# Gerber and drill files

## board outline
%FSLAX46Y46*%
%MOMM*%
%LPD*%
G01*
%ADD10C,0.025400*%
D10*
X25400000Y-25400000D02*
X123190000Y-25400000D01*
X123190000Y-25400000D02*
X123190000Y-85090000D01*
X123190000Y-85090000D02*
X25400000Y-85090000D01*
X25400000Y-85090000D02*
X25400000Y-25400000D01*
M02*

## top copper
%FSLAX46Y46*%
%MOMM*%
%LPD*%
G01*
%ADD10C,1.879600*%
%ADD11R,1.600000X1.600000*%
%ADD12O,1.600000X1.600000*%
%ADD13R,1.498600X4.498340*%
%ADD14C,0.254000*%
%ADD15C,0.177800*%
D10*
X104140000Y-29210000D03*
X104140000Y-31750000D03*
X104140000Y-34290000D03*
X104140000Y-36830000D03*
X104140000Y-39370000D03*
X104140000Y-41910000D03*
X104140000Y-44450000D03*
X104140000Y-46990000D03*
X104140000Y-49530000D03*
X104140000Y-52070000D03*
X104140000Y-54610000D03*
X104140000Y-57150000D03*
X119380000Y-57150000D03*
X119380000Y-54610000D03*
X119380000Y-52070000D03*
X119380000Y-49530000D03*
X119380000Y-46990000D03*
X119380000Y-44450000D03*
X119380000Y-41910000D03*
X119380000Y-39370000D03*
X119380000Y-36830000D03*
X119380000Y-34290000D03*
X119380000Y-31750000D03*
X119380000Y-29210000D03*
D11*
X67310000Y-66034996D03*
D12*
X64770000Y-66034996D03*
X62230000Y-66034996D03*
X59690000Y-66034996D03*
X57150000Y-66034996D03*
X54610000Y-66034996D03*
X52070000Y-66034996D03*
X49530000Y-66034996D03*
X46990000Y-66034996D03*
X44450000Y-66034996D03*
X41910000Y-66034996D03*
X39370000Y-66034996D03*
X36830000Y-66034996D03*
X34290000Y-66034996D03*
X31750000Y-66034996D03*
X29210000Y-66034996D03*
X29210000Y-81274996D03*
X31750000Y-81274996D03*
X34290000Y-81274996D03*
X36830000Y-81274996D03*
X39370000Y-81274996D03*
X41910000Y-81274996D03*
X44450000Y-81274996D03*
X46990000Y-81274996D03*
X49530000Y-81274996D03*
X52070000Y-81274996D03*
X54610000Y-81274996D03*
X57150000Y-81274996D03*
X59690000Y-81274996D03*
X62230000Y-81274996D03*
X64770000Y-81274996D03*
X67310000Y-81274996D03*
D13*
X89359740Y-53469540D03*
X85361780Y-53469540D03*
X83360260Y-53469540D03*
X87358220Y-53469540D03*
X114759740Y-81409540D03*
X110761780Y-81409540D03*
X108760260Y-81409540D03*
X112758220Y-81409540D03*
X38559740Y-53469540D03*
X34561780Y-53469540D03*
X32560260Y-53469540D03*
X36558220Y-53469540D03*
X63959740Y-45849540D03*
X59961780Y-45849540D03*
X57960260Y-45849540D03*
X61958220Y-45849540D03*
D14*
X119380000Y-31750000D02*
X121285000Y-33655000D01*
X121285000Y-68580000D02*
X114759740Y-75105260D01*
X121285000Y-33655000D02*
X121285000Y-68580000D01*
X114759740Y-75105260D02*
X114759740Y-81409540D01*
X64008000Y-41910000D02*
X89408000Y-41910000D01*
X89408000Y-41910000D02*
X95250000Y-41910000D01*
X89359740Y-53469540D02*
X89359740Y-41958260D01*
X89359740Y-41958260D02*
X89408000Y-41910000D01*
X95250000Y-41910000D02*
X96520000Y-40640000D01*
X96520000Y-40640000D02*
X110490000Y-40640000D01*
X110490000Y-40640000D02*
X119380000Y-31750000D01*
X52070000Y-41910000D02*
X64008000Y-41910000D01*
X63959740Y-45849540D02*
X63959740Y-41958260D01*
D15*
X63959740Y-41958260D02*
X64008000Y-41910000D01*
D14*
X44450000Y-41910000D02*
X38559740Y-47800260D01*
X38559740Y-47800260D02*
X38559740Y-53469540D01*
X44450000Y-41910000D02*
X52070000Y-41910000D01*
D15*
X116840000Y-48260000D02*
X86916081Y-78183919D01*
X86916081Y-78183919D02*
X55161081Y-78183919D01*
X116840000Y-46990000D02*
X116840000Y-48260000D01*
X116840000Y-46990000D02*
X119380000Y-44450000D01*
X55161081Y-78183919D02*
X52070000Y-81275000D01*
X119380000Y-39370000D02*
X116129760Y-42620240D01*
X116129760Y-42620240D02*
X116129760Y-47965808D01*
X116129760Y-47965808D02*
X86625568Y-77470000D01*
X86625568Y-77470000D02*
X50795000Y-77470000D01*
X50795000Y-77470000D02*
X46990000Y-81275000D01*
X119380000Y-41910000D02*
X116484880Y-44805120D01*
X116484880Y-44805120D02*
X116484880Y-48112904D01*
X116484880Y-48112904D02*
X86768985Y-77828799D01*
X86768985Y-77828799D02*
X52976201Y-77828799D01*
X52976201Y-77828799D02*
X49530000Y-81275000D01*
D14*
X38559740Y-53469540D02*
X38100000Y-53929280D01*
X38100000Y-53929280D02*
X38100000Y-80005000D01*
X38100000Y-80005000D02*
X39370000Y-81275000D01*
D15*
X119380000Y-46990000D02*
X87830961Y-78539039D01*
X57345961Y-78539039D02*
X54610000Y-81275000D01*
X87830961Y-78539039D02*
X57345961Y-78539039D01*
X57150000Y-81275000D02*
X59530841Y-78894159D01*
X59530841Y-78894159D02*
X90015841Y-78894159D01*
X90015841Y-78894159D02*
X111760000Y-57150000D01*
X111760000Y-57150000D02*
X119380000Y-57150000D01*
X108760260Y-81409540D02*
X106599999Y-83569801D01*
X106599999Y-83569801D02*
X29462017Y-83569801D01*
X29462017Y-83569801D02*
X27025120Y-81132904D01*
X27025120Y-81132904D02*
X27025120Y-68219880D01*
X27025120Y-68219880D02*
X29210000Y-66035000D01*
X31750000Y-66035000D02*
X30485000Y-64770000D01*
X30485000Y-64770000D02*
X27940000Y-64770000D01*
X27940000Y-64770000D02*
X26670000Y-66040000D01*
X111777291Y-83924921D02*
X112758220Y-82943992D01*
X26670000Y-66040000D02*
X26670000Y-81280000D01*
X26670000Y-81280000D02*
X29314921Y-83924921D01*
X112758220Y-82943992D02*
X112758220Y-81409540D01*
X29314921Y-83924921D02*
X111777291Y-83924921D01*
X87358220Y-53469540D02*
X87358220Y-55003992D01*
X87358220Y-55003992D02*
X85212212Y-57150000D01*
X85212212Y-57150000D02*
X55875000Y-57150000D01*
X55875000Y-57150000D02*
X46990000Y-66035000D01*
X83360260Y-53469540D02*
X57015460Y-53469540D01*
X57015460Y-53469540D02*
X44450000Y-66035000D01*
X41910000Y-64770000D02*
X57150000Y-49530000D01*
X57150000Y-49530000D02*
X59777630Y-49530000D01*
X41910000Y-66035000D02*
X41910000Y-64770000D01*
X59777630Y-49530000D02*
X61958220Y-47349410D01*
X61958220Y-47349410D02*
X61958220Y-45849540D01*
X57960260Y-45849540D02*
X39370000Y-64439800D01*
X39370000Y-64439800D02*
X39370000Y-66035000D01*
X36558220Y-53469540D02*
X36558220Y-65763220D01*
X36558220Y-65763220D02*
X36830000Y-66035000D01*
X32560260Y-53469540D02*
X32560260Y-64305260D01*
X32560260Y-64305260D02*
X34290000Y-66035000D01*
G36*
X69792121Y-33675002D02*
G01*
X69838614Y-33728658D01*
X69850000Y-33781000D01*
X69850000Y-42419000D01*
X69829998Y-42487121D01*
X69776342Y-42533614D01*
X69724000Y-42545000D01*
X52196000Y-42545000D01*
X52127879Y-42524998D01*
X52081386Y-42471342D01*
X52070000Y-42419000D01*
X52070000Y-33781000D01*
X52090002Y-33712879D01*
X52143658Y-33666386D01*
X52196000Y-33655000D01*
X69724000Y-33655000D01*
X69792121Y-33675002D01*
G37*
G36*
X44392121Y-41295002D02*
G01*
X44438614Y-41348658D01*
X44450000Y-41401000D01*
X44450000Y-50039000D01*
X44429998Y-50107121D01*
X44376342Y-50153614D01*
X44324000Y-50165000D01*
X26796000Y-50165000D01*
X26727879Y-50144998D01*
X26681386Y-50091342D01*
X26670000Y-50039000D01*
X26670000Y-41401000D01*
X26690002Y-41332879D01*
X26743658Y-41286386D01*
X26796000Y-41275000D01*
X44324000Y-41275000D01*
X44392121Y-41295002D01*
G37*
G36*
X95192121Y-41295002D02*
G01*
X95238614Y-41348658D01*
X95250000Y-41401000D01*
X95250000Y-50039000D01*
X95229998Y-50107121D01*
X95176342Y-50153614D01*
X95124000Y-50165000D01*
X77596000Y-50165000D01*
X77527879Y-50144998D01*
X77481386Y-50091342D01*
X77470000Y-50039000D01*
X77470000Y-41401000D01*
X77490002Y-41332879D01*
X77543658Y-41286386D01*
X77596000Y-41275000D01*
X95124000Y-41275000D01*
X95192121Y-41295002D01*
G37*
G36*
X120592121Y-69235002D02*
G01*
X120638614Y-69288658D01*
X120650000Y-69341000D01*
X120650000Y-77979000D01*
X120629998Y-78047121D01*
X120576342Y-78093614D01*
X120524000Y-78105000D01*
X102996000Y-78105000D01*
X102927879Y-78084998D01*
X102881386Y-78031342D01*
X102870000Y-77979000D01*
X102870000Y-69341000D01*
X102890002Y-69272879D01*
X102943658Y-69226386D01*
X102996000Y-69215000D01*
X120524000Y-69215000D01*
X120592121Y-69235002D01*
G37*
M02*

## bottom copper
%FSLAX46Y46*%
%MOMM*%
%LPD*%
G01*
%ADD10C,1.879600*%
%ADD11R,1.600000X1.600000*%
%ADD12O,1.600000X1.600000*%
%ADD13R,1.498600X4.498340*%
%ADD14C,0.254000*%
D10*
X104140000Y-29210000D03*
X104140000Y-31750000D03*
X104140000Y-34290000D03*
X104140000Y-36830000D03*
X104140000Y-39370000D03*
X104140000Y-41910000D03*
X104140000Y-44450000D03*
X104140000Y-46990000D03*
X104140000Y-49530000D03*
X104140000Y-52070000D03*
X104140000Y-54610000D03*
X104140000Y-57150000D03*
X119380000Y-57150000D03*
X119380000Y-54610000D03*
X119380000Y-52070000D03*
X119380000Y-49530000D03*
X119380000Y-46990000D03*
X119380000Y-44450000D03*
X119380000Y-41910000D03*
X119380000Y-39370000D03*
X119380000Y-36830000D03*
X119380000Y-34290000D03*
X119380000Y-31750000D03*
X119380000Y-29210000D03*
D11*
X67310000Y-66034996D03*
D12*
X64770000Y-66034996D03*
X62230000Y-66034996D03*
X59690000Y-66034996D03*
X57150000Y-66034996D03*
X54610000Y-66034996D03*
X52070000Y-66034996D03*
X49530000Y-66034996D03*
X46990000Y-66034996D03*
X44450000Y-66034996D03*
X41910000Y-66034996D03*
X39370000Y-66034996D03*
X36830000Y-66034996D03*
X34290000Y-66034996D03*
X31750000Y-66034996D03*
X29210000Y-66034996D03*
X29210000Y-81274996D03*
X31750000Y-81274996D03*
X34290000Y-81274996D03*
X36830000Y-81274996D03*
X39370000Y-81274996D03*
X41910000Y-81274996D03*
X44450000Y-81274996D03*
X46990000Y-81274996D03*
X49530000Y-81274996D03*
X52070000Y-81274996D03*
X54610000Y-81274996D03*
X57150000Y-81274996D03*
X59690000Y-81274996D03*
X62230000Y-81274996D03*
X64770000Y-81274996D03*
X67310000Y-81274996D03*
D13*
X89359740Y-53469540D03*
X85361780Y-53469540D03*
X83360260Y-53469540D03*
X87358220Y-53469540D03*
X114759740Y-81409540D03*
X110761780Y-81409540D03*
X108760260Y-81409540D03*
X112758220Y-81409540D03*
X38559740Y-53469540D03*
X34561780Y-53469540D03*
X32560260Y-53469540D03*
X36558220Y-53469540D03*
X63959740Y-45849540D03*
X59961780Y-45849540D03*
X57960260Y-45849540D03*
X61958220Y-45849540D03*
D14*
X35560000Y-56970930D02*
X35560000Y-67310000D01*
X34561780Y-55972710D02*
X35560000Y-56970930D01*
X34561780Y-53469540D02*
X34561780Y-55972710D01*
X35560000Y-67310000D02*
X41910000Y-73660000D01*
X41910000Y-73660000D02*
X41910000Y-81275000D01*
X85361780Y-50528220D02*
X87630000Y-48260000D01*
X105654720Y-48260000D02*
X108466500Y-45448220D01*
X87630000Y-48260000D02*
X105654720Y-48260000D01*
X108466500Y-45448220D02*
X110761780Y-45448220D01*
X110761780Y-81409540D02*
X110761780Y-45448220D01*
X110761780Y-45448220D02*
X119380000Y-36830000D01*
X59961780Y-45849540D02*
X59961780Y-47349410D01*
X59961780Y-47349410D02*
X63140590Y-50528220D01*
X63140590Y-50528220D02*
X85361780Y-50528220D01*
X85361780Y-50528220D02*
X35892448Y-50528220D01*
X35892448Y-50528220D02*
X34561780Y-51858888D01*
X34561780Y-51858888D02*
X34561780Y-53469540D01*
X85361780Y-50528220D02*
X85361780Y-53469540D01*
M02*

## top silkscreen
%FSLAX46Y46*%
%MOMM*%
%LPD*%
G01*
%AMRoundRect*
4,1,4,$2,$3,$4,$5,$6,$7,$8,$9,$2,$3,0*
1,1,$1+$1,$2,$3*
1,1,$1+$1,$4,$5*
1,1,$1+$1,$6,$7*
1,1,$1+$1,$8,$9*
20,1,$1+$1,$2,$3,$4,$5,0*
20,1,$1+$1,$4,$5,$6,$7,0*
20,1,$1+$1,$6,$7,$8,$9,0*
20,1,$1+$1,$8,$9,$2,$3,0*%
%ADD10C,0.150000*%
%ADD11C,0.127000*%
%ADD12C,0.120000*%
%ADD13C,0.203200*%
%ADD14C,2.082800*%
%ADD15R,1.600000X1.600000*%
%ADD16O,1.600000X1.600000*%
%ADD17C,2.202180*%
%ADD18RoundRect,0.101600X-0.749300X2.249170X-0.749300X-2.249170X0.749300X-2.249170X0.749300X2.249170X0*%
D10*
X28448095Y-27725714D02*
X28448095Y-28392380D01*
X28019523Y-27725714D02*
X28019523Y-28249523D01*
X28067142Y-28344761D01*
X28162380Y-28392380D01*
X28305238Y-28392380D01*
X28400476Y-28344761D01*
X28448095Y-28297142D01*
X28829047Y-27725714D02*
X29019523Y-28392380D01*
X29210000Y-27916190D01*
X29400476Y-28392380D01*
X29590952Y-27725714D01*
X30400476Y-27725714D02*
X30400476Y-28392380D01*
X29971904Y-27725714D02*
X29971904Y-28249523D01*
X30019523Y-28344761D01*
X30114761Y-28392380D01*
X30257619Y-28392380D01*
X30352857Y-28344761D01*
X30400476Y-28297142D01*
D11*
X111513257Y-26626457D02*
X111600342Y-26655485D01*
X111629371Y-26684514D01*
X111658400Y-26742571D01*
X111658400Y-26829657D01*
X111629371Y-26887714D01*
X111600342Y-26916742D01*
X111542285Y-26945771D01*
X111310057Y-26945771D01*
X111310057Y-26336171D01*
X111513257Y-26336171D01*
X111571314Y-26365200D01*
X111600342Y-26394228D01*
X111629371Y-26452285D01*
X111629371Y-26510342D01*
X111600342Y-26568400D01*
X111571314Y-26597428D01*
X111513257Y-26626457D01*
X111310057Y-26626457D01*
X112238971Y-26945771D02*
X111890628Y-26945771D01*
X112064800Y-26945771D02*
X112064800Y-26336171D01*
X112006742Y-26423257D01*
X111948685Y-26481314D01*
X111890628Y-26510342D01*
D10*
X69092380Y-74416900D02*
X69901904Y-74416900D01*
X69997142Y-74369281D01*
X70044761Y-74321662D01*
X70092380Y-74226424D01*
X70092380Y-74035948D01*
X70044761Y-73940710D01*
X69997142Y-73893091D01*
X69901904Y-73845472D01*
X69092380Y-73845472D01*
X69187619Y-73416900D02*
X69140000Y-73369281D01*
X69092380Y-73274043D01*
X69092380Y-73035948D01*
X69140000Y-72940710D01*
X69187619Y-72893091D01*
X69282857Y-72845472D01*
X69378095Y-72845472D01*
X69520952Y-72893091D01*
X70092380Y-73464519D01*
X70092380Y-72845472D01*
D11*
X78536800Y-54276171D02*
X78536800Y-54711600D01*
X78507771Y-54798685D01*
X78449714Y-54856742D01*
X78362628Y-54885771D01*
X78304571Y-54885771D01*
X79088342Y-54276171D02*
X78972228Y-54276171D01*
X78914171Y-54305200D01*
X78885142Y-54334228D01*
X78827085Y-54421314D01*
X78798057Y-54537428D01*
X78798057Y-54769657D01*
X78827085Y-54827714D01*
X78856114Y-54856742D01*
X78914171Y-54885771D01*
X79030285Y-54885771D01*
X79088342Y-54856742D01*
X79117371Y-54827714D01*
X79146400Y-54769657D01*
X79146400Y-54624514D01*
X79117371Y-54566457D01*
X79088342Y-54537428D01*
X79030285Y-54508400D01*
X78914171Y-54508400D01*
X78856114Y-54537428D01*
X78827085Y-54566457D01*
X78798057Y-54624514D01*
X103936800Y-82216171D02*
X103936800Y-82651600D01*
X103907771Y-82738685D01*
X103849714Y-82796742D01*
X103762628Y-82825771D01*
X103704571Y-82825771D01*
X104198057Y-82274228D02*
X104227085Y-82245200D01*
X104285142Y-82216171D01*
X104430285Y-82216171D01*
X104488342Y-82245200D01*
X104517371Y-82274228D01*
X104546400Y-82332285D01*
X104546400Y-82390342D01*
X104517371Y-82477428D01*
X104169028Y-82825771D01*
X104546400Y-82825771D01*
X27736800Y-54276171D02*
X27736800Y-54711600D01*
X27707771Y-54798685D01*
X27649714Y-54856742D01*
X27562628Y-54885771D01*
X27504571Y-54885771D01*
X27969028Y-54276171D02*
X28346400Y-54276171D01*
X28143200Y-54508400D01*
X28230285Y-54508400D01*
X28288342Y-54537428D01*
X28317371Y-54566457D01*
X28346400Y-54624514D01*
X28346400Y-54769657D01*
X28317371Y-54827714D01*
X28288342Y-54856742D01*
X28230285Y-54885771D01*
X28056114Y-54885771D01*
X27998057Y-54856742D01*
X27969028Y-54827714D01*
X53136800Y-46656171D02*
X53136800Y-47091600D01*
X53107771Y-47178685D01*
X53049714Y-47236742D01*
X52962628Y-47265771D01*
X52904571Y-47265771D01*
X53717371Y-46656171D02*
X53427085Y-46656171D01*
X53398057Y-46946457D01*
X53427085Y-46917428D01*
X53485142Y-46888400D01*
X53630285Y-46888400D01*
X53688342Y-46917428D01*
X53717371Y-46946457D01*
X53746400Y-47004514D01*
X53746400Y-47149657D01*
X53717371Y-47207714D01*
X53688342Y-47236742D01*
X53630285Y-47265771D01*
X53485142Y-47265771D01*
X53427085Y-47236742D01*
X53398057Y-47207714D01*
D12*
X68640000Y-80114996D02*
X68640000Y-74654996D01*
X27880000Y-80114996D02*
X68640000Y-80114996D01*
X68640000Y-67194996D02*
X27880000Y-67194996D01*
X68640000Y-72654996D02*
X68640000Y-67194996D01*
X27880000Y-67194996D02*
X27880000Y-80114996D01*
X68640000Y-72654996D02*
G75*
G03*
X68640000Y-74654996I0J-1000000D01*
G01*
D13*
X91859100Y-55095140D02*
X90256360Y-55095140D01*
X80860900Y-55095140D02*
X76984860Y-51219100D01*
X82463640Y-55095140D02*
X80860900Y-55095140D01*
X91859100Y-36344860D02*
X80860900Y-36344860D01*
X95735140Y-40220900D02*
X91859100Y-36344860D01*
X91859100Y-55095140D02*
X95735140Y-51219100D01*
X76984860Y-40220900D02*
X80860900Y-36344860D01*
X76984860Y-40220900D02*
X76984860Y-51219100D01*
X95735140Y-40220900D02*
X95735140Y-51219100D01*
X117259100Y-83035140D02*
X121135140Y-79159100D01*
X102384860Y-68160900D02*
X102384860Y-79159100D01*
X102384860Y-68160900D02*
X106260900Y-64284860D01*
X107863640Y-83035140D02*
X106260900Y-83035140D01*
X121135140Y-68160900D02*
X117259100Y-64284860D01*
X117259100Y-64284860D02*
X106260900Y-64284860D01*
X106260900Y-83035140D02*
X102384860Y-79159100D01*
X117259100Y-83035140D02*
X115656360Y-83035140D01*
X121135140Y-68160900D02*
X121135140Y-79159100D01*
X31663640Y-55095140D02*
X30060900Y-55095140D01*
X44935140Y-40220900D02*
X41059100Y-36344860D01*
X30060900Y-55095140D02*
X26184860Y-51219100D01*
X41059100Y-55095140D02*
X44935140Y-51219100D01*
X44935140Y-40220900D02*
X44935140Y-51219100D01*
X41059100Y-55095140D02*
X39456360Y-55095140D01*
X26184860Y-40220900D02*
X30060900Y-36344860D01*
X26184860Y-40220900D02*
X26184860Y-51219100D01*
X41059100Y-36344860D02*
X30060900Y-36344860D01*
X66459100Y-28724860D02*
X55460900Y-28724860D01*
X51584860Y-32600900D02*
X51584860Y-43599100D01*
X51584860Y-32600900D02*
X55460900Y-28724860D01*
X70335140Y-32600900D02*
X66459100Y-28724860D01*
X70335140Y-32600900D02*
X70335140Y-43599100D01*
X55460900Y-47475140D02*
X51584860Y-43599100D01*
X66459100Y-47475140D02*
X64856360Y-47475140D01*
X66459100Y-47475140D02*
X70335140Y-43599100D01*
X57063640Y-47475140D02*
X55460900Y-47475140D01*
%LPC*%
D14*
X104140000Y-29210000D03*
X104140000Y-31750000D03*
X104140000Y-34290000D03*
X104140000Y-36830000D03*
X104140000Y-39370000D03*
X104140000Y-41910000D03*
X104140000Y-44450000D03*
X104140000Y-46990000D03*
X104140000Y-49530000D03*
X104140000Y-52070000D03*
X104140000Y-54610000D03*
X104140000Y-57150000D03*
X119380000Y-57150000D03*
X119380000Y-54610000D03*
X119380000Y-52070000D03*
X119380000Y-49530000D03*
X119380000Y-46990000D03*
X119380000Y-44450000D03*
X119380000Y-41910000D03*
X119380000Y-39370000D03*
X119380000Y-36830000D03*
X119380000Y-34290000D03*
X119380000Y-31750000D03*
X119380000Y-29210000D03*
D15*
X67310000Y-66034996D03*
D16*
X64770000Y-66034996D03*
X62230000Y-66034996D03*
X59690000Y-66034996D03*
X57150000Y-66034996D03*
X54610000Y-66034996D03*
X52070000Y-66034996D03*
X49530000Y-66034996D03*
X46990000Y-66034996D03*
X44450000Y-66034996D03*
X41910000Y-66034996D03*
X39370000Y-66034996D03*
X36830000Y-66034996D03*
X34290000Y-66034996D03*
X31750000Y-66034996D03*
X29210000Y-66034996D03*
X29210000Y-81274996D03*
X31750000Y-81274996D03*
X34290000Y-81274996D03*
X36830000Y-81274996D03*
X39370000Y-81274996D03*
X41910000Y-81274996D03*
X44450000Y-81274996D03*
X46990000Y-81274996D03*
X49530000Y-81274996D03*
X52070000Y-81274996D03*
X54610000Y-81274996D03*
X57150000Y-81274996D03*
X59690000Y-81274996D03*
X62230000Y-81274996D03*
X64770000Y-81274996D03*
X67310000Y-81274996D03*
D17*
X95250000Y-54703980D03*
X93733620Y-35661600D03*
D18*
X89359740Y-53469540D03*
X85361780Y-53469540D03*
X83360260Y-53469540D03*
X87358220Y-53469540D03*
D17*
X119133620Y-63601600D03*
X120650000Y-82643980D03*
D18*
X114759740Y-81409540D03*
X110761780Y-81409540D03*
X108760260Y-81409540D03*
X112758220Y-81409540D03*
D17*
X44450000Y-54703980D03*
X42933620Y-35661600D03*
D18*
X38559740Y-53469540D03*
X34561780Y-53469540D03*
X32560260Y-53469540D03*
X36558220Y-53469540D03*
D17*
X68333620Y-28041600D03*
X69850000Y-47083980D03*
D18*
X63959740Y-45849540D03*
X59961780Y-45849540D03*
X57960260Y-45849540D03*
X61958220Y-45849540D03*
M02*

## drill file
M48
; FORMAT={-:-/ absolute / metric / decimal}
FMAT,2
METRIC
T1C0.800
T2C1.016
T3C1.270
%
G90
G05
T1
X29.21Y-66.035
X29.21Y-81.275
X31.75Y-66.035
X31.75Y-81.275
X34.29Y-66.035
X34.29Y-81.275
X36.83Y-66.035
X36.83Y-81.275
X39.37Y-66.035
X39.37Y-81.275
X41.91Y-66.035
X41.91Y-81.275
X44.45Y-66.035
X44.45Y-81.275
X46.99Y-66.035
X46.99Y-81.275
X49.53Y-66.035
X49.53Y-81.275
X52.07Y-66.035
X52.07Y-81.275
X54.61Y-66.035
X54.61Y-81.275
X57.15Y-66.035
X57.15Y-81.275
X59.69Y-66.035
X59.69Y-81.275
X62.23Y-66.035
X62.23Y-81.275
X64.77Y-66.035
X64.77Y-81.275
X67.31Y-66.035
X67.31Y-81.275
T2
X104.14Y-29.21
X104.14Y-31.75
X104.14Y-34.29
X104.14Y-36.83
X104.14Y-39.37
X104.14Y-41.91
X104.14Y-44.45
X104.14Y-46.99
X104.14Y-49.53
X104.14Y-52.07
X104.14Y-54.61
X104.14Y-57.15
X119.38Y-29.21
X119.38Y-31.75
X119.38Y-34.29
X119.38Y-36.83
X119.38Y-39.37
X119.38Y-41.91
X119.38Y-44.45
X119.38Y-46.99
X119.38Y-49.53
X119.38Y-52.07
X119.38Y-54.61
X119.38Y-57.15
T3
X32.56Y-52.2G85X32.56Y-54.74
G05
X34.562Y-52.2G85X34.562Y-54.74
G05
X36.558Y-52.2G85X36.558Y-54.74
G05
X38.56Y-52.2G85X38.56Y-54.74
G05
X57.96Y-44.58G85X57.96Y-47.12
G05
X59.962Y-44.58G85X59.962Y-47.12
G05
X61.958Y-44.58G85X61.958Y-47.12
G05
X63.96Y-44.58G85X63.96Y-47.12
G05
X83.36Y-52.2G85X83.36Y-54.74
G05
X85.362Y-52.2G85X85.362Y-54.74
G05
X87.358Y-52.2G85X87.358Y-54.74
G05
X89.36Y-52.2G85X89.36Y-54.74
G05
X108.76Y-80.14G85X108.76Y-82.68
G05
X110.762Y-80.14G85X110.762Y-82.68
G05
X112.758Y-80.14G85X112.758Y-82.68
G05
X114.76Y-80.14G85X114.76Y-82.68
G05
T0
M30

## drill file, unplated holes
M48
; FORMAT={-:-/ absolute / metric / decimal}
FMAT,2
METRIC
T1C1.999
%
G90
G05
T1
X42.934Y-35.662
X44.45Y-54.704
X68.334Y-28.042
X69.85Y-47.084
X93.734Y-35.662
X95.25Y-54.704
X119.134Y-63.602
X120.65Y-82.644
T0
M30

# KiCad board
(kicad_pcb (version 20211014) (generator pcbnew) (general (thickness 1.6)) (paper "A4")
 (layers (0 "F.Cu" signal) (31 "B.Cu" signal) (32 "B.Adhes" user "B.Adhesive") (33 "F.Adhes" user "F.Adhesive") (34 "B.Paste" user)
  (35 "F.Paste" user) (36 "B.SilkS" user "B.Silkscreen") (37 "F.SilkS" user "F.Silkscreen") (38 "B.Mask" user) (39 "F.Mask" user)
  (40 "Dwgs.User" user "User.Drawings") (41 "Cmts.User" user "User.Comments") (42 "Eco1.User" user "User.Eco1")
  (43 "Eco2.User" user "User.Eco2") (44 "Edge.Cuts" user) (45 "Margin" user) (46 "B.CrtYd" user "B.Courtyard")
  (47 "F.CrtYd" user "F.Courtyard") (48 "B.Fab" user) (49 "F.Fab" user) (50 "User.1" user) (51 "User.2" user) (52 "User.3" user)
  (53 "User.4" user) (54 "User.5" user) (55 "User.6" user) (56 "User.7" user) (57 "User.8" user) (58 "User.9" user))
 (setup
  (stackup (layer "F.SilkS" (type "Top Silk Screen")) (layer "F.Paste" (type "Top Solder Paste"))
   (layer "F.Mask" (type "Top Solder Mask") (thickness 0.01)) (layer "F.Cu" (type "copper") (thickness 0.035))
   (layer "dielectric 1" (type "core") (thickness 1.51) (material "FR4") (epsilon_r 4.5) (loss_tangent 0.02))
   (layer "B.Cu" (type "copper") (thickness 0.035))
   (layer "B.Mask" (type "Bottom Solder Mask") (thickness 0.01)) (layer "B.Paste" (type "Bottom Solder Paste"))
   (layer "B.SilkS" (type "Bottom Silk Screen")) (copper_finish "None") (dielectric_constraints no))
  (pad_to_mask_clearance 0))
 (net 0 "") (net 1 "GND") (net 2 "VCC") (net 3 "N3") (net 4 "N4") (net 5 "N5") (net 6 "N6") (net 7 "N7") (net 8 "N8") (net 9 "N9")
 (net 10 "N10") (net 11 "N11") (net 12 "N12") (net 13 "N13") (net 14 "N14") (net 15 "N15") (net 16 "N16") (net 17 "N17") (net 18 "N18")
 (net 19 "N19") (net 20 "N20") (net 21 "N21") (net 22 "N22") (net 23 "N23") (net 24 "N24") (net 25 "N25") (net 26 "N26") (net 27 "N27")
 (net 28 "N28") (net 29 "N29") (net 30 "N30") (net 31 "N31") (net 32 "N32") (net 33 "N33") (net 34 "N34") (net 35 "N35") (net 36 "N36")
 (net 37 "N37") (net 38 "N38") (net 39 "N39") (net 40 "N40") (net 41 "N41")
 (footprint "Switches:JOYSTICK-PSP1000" (layer "F.Cu") (at 111.76 73.66 180)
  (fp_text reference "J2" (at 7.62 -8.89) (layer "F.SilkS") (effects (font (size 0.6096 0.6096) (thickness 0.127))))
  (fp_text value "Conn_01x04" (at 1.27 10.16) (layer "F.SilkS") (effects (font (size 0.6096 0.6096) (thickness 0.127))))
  (fp_line (start -5.4991 -9.37514) (end -9.37514 -5.4991) (layer "F.SilkS") (width 0.2032))
  (fp_line (start 9.37514 5.4991) (end 9.37514 -5.4991) (layer "F.SilkS") (width 0.2032))
  (fp_line (start 9.37514 5.4991) (end 5.4991 9.37514) (layer "F.SilkS") (width 0.2032))
  (fp_line (start 3.89636 -9.37514) (end 5.4991 -9.37514) (layer "F.SilkS") (width 0.2032))
  (fp_line (start -9.37514 5.4991) (end -5.4991 9.37514) (layer "F.SilkS") (width 0.2032))
  (fp_line (start -5.4991 9.37514) (end 5.4991 9.37514) (layer "F.SilkS") (width 0.2032))
  (fp_line (start 5.4991 -9.37514) (end 9.37514 -5.4991) (layer "F.SilkS") (width 0.2032))
  (fp_line (start -5.4991 -9.37514) (end -3.89636 -9.37514) (layer "F.SilkS") (width 0.2032))
  (fp_line (start -9.37514 5.4991) (end -9.37514 -5.4991) (layer "F.SilkS") (width 0.2032))
  (pad "" np_thru_hole circle (at -7.37362 10.0584 180) (size 1.99898 1.99898) (drill 1.99898) (layers *.Cu *.Mask)
   (solder_mask_margin 0.1016))
  (pad "" np_thru_hole circle (at -8.89 -8.98398 180) (size 1.99898 1.99898) (drill 1.99898) (layers *.Cu *.Mask)
   (solder_mask_margin 0.1016))
  (pad "GND" thru_hole rect (at -2.99974 -7.74954 270) (size 4.49834 1.4986) (drill oval 3.81 1.27) (layers *.Cu *.Mask) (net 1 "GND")
   (solder_mask_margin 0.1016))
  (pad "VCC" thru_hole rect (at 0.99822 -7.74954 270) (size 4.49834 1.4986) (drill oval 3.81 1.27) (layers *.Cu *.Mask) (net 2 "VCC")
   (solder_mask_margin 0.1016))
  (pad "X" thru_hole rect (at 2.99974 -7.74954 270) (size 4.49834 1.4986) (drill oval 3.81 1.27) (layers *.Cu *.Mask) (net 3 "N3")
   (solder_mask_margin 0.1016))
  (pad "Y" thru_hole rect (at -0.99822 -7.74954 270) (size 4.49834 1.4986) (drill oval 3.81 1.27) (layers *.Cu *.Mask) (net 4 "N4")
   (solder_mask_margin 0.1016)))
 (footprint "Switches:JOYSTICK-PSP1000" (layer "F.Cu") (at 86.36 45.72 180)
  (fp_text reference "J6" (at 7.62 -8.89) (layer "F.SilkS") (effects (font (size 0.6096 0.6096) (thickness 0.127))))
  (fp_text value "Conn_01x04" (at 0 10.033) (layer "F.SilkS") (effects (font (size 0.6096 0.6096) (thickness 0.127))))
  (fp_line (start -5.4991 -9.37514) (end -3.89636 -9.37514) (layer "F.SilkS") (width 0.2032))
  (fp_line (start 5.4991 -9.37514) (end 9.37514 -5.4991) (layer "F.SilkS") (width 0.2032))
  (fp_line (start 3.89636 -9.37514) (end 5.4991 -9.37514) (layer "F.SilkS") (width 0.2032))
  (fp_line (start -5.4991 9.37514) (end 5.4991 9.37514) (layer "F.SilkS") (width 0.2032))
  (fp_line (start -9.37514 5.4991) (end -5.4991 9.37514) (layer "F.SilkS") (width 0.2032))
  (fp_line (start -5.4991 -9.37514) (end -9.37514 -5.4991) (layer "F.SilkS") (width 0.2032))
  (fp_line (start 9.37514 5.4991) (end 5.4991 9.37514) (layer "F.SilkS") (width 0.2032))
  (fp_line (start 9.37514 5.4991) (end 9.37514 -5.4991) (layer "F.SilkS") (width 0.2032))
  (fp_line (start -9.37514 5.4991) (end -9.37514 -5.4991) (layer "F.SilkS") (width 0.2032))
  (pad "" np_thru_hole circle locked (at -8.89 -8.98398 180) (size 1.99898 1.99898) (drill 1.99898) (layers *.Cu *.Mask)
   (solder_mask_margin 0.1016))
  (pad "" np_thru_hole circle locked (at -7.37362 10.0584 180) (size 1.99898 1.99898) (drill 1.99898) (layers *.Cu *.Mask)
   (solder_mask_margin 0.1016))
  (pad "GND" thru_hole rect locked (at -2.99974 -7.74954 270) (size 4.49834 1.4986) (drill oval 3.81 1.27) (layers *.Cu *.Mask)
   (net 1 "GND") (solder_mask_margin 0.1016))
  (pad "VCC" thru_hole rect locked (at 0.99822 -7.74954 270) (size 4.49834 1.4986) (drill oval 3.81 1.27) (layers *.Cu *.Mask) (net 2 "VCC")
   (solder_mask_margin 0.1016))
  (pad "X" thru_hole rect locked (at 2.99974 -7.74954 270) (size 4.49834 1.4986) (drill oval 3.81 1.27) (layers *.Cu *.Mask) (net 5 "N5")
   (solder_mask_margin 0.1016))
  (pad "Y" thru_hole rect locked (at -0.99822 -7.74954 270) (size 4.49834 1.4986) (drill oval 3.81 1.27) (layers *.Cu *.Mask) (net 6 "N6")
   (solder_mask_margin 0.1016)))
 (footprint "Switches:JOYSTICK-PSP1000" (layer "F.Cu") (at 35.56 45.72 180)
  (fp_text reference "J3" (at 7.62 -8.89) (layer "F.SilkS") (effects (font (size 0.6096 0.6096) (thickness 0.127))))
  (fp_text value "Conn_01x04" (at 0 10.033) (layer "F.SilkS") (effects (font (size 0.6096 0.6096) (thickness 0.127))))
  (fp_line (start 3.89636 -9.37514) (end 5.4991 -9.37514) (layer "F.SilkS") (width 0.2032))
  (fp_line (start -9.37514 5.4991) (end -5.4991 9.37514) (layer "F.SilkS") (width 0.2032))
  (fp_line (start 5.4991 -9.37514) (end 9.37514 -5.4991) (layer "F.SilkS") (width 0.2032))
  (fp_line (start -5.4991 -9.37514) (end -9.37514 -5.4991) (layer "F.SilkS") (width 0.2032))
  (fp_line (start -9.37514 5.4991) (end -9.37514 -5.4991) (layer "F.SilkS") (width 0.2032))
  (fp_line (start -5.4991 -9.37514) (end -3.89636 -9.37514) (layer "F.SilkS") (width 0.2032))
  (fp_line (start 9.37514 5.4991) (end 5.4991 9.37514) (layer "F.SilkS") (width 0.2032))
  (fp_line (start 9.37514 5.4991) (end 9.37514 -5.4991) (layer "F.SilkS") (width 0.2032))
  (fp_line (start -5.4991 9.37514) (end 5.4991 9.37514) (layer "F.SilkS") (width 0.2032))
  (pad "" np_thru_hole circle locked (at -8.89 -8.98398 180) (size 1.99898 1.99898) (drill 1.99898) (layers *.Cu *.Mask)
   (solder_mask_margin 0.1016))
  (pad "" np_thru_hole circle locked (at -7.37362 10.0584 180) (size 1.99898 1.99898) (drill 1.99898) (layers *.Cu *.Mask)
   (solder_mask_margin 0.1016))
  (pad "GND" thru_hole rect locked (at -2.99974 -7.74954 270) (size 4.49834 1.4986) (drill oval 3.81 1.27) (layers *.Cu *.Mask)
   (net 1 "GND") (solder_mask_margin 0.1016))
  (pad "VCC" thru_hole rect locked (at 0.99822 -7.74954 270) (size 4.49834 1.4986) (drill oval 3.81 1.27) (layers *.Cu *.Mask) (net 2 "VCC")
   (solder_mask_margin 0.1016))
  (pad "X" thru_hole rect locked (at 2.99974 -7.74954 270) (size 4.49834 1.4986) (drill oval 3.81 1.27) (layers *.Cu *.Mask) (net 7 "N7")
   (solder_mask_margin 0.1016))
  (pad "Y" thru_hole rect locked (at -0.99822 -7.74954 270) (size 4.49834 1.4986) (drill oval 3.81 1.27) (layers *.Cu *.Mask) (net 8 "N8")
   (solder_mask_margin 0.1016)))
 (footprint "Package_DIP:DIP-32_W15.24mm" (layer "F.Cu") (at 67.31 66.034996 -90)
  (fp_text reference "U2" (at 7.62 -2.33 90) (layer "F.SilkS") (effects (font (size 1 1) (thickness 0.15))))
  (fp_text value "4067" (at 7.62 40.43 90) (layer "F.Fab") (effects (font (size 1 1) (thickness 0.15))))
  (fp_line (start 1.16 39.43) (end 14.08 39.43) (layer "F.SilkS") (width 0.12))
  (fp_line (start 14.08 39.43) (end 14.08 -1.33) (layer "F.SilkS") (width 0.12))
  (fp_line (start 6.62 -1.33) (end 1.16 -1.33) (layer "F.SilkS") (width 0.12))
  (fp_line (start 14.08 -1.33) (end 8.62 -1.33) (layer "F.SilkS") (width 0.12))
  (fp_line (start 1.16 -1.33) (end 1.16 39.43) (layer "F.SilkS") (width 0.12))
  (fp_arc (start 8.62 -1.33) (mid 7.62 -0.33) (end 6.62 -1.33) (layer "F.SilkS") (width 0.12))
  (pad "0" thru_hole oval (at 15.24 35.56 270) (size 1.6 1.6) (drill 0.8) (layers *.Cu *.Mask))
  (pad "0" thru_hole oval (at 15.24 7.62 270) (size 1.6 1.6) (drill 0.8) (layers *.Cu *.Mask))
  (pad "0" thru_hole oval (at 15.24 5.08 270) (size 1.6 1.6) (drill 0.8) (layers *.Cu *.Mask))
  (pad "0" thru_hole oval (at 15.24 2.54 270) (size 1.6 1.6) (drill 0.8) (layers *.Cu *.Mask))
  (pad "0" thru_hole oval (at 15.24 33.02 270) (size 1.6 1.6) (drill 0.8) (layers *.Cu *.Mask))
  (pad "0" thru_hole oval (at 15.24 30.48 270) (size 1.6 1.6) (drill 0.8) (layers *.Cu *.Mask))
  (pad "0" thru_hole oval (at 15.24 0 270) (size 1.6 1.6) (drill 0.8) (layers *.Cu *.Mask))
  (pad "0" thru_hole oval (at 15.24 38.1 270) (size 1.6 1.6) (drill 0.8) (layers *.Cu *.Mask))
  (pad "1" thru_hole oval (at 15.24 10.16 270) (size 1.6 1.6) (drill 0.8) (layers *.Cu *.Mask) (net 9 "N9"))
  (pad "2" thru_hole oval (at 0 20.32 270) (size 1.6 1.6) (drill 0.8) (layers *.Cu *.Mask) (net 6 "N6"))
  (pad "3" thru_hole oval (at 0 22.86 270) (size 1.6 1.6) (drill 0.8) (layers *.Cu *.Mask) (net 5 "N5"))
  (pad "4" thru_hole oval (at 0 25.4 270) (size 1.6 1.6) (drill 0.8) (layers *.Cu *.Mask) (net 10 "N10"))
  (pad "5" thru_hole oval (at 0 27.94 270) (size 1.6 1.6) (drill 0.8) (layers *.Cu *.Mask) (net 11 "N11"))
  (pad "6" thru_hole oval (at 0 30.48 270) (size 1.6 1.6) (drill 0.8) (layers *.Cu *.Mask) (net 8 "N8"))
  (pad "7" thru_hole oval (at 0 33.02 270) (size 1.6 1.6) (drill 0.8) (layers *.Cu *.Mask) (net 7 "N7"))
  (pad "8" thru_hole oval (at 0 35.56 270) (size 1.6 1.6) (drill 0.8) (layers *.Cu *.Mask) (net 4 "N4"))
  (pad "9" thru_hole oval (at 0 38.1 270) (size 1.6 1.6) (drill 0.8) (layers *.Cu *.Mask) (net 3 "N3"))
  (pad "10" thru_hole oval (at 15.24 20.32 270) (size 1.6 1.6) (drill 0.8) (layers *.Cu *.Mask) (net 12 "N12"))
  (pad "11" thru_hole oval (at 15.24 17.78 270) (size 1.6 1.6) (drill 0.8) (layers *.Cu *.Mask) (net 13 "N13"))
  (pad "12" thru_hole oval (at 15.24 27.94 270) (size 1.6 1.6) (drill 0.8) (layers *.Cu *.Mask) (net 1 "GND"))
  (pad "13" thru_hole oval (at 15.24 12.7 270) (size 1.6 1.6) (drill 0.8) (layers *.Cu *.Mask) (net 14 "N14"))
  (pad "14" thru_hole oval (at 15.24 15.24 270) (size 1.6 1.6) (drill 0.8) (layers *.Cu *.Mask) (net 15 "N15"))
  (pad "15" thru_hole oval (at 15.24 22.86 270) (size 1.6 1.6) (drill 0.8) (layers *.Cu *.Mask) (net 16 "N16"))
  (pad "16" thru_hole rect (at 0 0 270) (size 1.6 1.6) (drill 0.8) (layers *.Cu *.Mask) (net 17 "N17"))
  (pad "17" thru_hole oval (at 0 2.54 270) (size 1.6 1.6) (drill 0.8) (layers *.Cu *.Mask) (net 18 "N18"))
  (pad "18" thru_hole oval (at 0 5.08 270) (size 1.6 1.6) (drill 0.8) (layers *.Cu *.Mask) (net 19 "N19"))
  (pad "19" thru_hole oval (at 0 7.62 270) (size 1.6 1.6) (drill 0.8) (layers *.Cu *.Mask) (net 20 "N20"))
  (pad "20" thru_hole oval (at 0 10.16 270) (size 1.6 1.6) (drill 0.8) (layers *.Cu *.Mask) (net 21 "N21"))
  (pad "21" thru_hole oval (at 0 12.7 270) (size 1.6 1.6) (drill 0.8) (layers *.Cu *.Mask) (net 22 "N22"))
  (pad "22" thru_hole oval (at 0 15.24 270) (size 1.6 1.6) (drill 0.8) (layers *.Cu *.Mask) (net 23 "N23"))
  (pad "23" thru_hole oval (at 0 17.78 270) (size 1.6 1.6) (drill 0.8) (layers *.Cu *.Mask) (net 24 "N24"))
  (pad "24" thru_hole oval (at 15.24 25.4 270) (size 1.6 1.6) (drill 0.8) (layers *.Cu *.Mask) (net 2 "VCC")))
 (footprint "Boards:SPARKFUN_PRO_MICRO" (layer "F.Cu") (at 111.76 41.91)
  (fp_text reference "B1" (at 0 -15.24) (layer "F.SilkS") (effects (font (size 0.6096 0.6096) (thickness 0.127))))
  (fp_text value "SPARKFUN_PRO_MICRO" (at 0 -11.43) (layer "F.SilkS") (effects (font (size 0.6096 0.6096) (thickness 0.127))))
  (pad "1" thru_hole circle locked (at -7.62 -12.7) (size 1.8796 1.8796) (drill 1.016) (layers *.Cu *.Mask) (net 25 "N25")
   (solder_mask_margin 0.1016))
  (pad "2" thru_hole circle locked (at -7.62 -10.16) (size 1.8796 1.8796) (drill 1.016) (layers *.Cu *.Mask) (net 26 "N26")
   (solder_mask_margin 0.1016))
  (pad "3" thru_hole circle locked (at -7.62 -7.62) (size 1.8796 1.8796) (drill 1.016) (layers *.Cu *.Mask) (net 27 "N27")
   (solder_mask_margin 0.1016))
  (pad "4" thru_hole circle locked (at -7.62 -5.08) (size 1.8796 1.8796) (drill 1.016) (layers *.Cu *.Mask) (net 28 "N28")
   (solder_mask_margin 0.1016))
  (pad "5" thru_hole circle locked (at -7.62 -2.54) (size 1.8796 1.8796) (drill 1.016) (layers *.Cu *.Mask) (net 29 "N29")
   (solder_mask_margin 0.1016))
  (pad "6" thru_hole circle locked (at -7.62 0) (size 1.8796 1.8796) (drill 1.016) (layers *.Cu *.Mask) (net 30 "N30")
   (solder_mask_margin 0.1016))
  (pad "7" thru_hole circle locked (at -7.62 2.54) (size 1.8796 1.8796) (drill 1.016) (layers *.Cu *.Mask) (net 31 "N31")
   (solder_mask_margin 0.1016))
  (pad "8" thru_hole circle locked (at -7.62 5.08) (size 1.8796 1.8796) (drill 1.016) (layers *.Cu *.Mask) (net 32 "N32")
   (solder_mask_margin 0.1016))
  (pad "9" thru_hole circle locked (at -7.62 7.62) (size 1.8796 1.8796) (drill 1.016) (layers *.Cu *.Mask) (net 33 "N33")
   (solder_mask_margin 0.1016))
  (pad "10" thru_hole circle locked (at -7.62 10.16) (size 1.8796 1.8796) (drill 1.016) (layers *.Cu *.Mask) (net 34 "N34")
   (solder_mask_margin 0.1016))
  (pad "11" thru_hole circle locked (at -7.62 12.7) (size 1.8796 1.8796) (drill 1.016) (layers *.Cu *.Mask) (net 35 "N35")
   (solder_mask_margin 0.1016))
  (pad "12" thru_hole circle locked (at -7.62 15.24) (size 1.8796 1.8796) (drill 1.016) (layers *.Cu *.Mask) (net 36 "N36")
   (solder_mask_margin 0.1016))
  (pad "13" thru_hole circle locked (at 7.62 15.24) (size 1.8796 1.8796) (drill 1.016) (layers *.Cu *.Mask) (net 9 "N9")
   (solder_mask_margin 0.1016))
  (pad "14" thru_hole circle locked (at 7.62 12.7) (size 1.8796 1.8796) (drill 1.016) (layers *.Cu *.Mask) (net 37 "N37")
   (solder_mask_margin 0.1016))
  (pad "15" thru_hole circle locked (at 7.62 10.16) (size 1.8796 1.8796) (drill 1.016) (layers *.Cu *.Mask) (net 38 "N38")
   (solder_mask_margin 0.1016))
  (pad "16" thru_hole circle locked (at 7.62 7.62) (size 1.8796 1.8796) (drill 1.016) (layers *.Cu *.Mask) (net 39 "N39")
   (solder_mask_margin 0.1016))
  (pad "17" thru_hole circle locked (at 7.62 5.08) (size 1.8796 1.8796) (drill 1.016) (layers *.Cu *.Mask) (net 14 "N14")
   (solder_mask_margin 0.1016))
  (pad "18" thru_hole circle locked (at 7.62 2.54) (size 1.8796 1.8796) (drill 1.016) (layers *.Cu *.Mask) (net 15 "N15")
   (solder_mask_margin 0.1016))
  (pad "19" thru_hole circle locked (at 7.62 0) (size 1.8796 1.8796) (drill 1.016) (layers *.Cu *.Mask) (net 13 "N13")
   (solder_mask_margin 0.1016))
  (pad "20" thru_hole circle locked (at 7.62 -2.54) (size 1.8796 1.8796) (drill 1.016) (layers *.Cu *.Mask) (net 12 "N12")
   (solder_mask_margin 0.1016))
  (pad "21" thru_hole circle locked (at 7.62 -5.08) (size 1.8796 1.8796) (drill 1.016) (layers *.Cu *.Mask) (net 2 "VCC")
   (solder_mask_margin 0.1016))
  (pad "22" thru_hole circle locked (at 7.62 -7.62) (size 1.8796 1.8796) (drill 1.016) (layers *.Cu *.Mask) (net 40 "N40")
   (solder_mask_margin 0.1016))
  (pad "23" thru_hole circle locked (at 7.62 -10.16) (size 1.8796 1.8796) (drill 1.016) (layers *.Cu *.Mask) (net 1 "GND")
   (solder_mask_margin 0.1016))
  (pad "24" thru_hole circle locked (at 7.62 -12.7) (size 1.8796 1.8796) (drill 1.016) (layers *.Cu *.Mask) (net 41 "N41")
   (solder_mask_margin 0.1016)))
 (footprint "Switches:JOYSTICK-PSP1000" (layer "F.Cu") (at 60.96 38.1 180)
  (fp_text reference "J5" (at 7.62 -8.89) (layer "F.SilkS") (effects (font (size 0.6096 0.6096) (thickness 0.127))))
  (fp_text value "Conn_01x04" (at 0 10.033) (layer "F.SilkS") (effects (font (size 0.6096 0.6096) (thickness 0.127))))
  (fp_line (start -5.4991 9.37514) (end 5.4991 9.37514) (layer "F.SilkS") (width 0.2032))
  (fp_line (start 9.37514 5.4991) (end 9.37514 -5.4991) (layer "F.SilkS") (width 0.2032))
  (fp_line (start 9.37514 5.4991) (end 5.4991 9.37514) (layer "F.SilkS") (width 0.2032))
  (fp_line (start -9.37514 5.4991) (end -5.4991 9.37514) (layer "F.SilkS") (width 0.2032))
  (fp_line (start -9.37514 5.4991) (end -9.37514 -5.4991) (layer "F.SilkS") (width 0.2032))
  (fp_line (start 5.4991 -9.37514) (end 9.37514 -5.4991) (layer "F.SilkS") (width 0.2032))
  (fp_line (start -5.4991 -9.37514) (end -3.89636 -9.37514) (layer "F.SilkS") (width 0.2032))
  (fp_line (start -5.4991 -9.37514) (end -9.37514 -5.4991) (layer "F.SilkS") (width 0.2032))
  (fp_line (start 3.89636 -9.37514) (end 5.4991 -9.37514) (layer "F.SilkS") (width 0.2032))
  (pad "" np_thru_hole circle locked (at -7.37362 10.0584 180) (size 1.99898 1.99898) (drill 1.99898) (layers *.Cu *.Mask)
   (solder_mask_margin 0.1016))
  (pad "" np_thru_hole circle locked (at -8.89 -8.98398 180) (size 1.99898 1.99898) (drill 1.99898) (layers *.Cu *.Mask)
   (solder_mask_margin 0.1016))
  (pad "GND" thru_hole rect locked (at -2.99974 -7.74954 270) (size 4.49834 1.4986) (drill oval 3.81 1.27) (layers *.Cu *.Mask)
   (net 1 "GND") (solder_mask_margin 0.1016))
  (pad "VCC" thru_hole rect locked (at 0.99822 -7.74954 270) (size 4.49834 1.4986) (drill oval 3.81 1.27) (layers *.Cu *.Mask) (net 2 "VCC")
   (solder_mask_margin 0.1016))
  (pad "X" thru_hole rect locked (at 2.99974 -7.74954 270) (size 4.49834 1.4986) (drill oval 3.81 1.27) (layers *.Cu *.Mask) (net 11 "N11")
   (solder_mask_margin 0.1016))
  (pad "Y" thru_hole rect locked (at -0.99822 -7.74954 270) (size 4.49834 1.4986) (drill oval 3.81 1.27) (layers *.Cu *.Mask) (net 10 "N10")
   (solder_mask_margin 0.1016)))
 (gr_rect (start 25.4 25.4) (end 123.19 85.09) (layer "Edge.Cuts") (width 0.0254) (fill none))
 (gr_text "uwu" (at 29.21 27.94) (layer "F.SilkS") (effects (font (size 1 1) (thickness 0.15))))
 (segment (start 41.91 73.66) (end 41.91 81.275) (width 0.254) (layer "B.Cu") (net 2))
 (segment (start 85.36178 50.52822) (end 35.892448 50.52822) (width 0.254) (layer "B.Cu") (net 2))
 (segment (start 35.56 67.31) (end 41.91 73.66) (width 0.254) (layer "B.Cu") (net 2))
 (segment (start 63.14059 50.52822) (end 85.36178 50.52822) (width 0.254) (layer "B.Cu") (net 2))
 (segment (start 108.4665 45.44822) (end 110.76178 45.44822) (width 0.254) (layer "B.Cu") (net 2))
 (segment (start 59.96178 47.34941) (end 63.14059 50.52822) (width 0.254) (layer "B.Cu") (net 2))
 (segment (start 110.76178 45.44822) (end 119.38 36.83) (width 0.254) (layer "B.Cu") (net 2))
 (segment (start 110.76178 81.40954) (end 110.76178 45.44822) (width 0.254) (layer "B.Cu") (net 2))
 (segment (start 85.36178 50.52822) (end 85.36178 53.46954) (width 0.254) (layer "B.Cu") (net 2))
 (segment (start 34.56178 51.858888) (end 34.56178 53.46954) (width 0.254) (layer "B.Cu") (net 2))
 (segment (start 34.56178 55.97271) (end 35.56 56.97093) (width 0.254) (layer "B.Cu") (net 2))
 (segment (start 34.56178 53.46954) (end 34.56178 55.97271) (width 0.254) (layer "B.Cu") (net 2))
 (segment (start 105.65472 48.26) (end 108.4665 45.44822) (width 0.254) (layer "B.Cu") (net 2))
 (segment (start 35.56 56.97093) (end 35.56 67.31) (width 0.254) (layer "B.Cu") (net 2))
 (segment (start 59.96178 45.84954) (end 59.96178 47.34941) (width 0.254) (layer "B.Cu") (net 2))
 (segment (start 85.36178 50.52822) (end 87.63 48.26) (width 0.254) (layer "B.Cu") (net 2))
 (segment (start 87.63 48.26) (end 105.65472 48.26) (width 0.254) (layer "B.Cu") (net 2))
 (segment (start 35.892448 50.52822) (end 34.56178 51.858888) (width 0.254) (layer "B.Cu") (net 2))
 (segment (start 121.285 68.58) (end 114.75974 75.10526) (width 0.254) (layer "F.Cu") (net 1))
 (segment (start 38.55974 53.46954) (end 38.1 53.92928) (width 0.254) (layer "F.Cu") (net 1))
 (segment (start 38.1 80.005) (end 39.37 81.275) (width 0.254) (layer "F.Cu") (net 1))
 (segment (start 119.38 31.75) (end 121.285 33.655) (width 0.254) (layer "F.Cu") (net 1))
 (segment (start 96.52 40.64) (end 110.49 40.64) (width 0.254) (layer "F.Cu") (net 1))
 (segment (start 89.35974 53.46954) (end 89.35974 41.95826) (width 0.254) (layer "F.Cu") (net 1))
 (segment (start 38.55974 47.80026) (end 38.55974 53.46954) (width 0.254) (layer "F.Cu") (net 1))
 (segment (start 89.35974 41.95826) (end 89.408 41.91) (width 0.254) (layer "F.Cu") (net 1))
 (segment (start 64.008 41.91) (end 89.408 41.91) (width 0.254) (layer "F.Cu") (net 1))
 (segment (start 114.75974 75.10526) (end 114.75974 81.40954) (width 0.254) (layer "F.Cu") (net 1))
 (segment (start 95.25 41.91) (end 96.52 40.64) (width 0.254) (layer "F.Cu") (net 1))
 (segment (start 44.45 41.91) (end 52.07 41.91) (width 0.254) (layer "F.Cu") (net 1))
 (segment (start 110.49 40.64) (end 119.38 31.75) (width 0.254) (layer "F.Cu") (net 1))
 (segment (start 63.95974 45.84954) (end 63.95974 41.95826) (width 0.254) (layer "F.Cu") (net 1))
 (segment (start 52.07 41.91) (end 64.008 41.91) (width 0.254) (layer "F.Cu") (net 1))
 (segment (start 121.285 33.655) (end 121.285 68.58) (width 0.254) (layer "F.Cu") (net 1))
 (segment (start 89.408 41.91) (end 95.25 41.91) (width 0.254) (layer "F.Cu") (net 1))
 (segment (start 63.95974 41.95826) (end 64.008 41.91) (width 0.1778) (layer "F.Cu") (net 1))
 (segment (start 44.45 41.91) (end 38.55974 47.80026) (width 0.254) (layer "F.Cu") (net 1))
 (segment (start 38.1 53.92928) (end 38.1 80.005) (width 0.254) (layer "F.Cu") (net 1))
 (segment (start 27.02512 81.132904) (end 27.02512 68.21988) (width 0.1778) (layer "F.Cu") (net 3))
 (segment (start 106.599999 83.569801) (end 29.462017 83.569801) (width 0.1778) (layer "F.Cu") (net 3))
 (segment (start 108.76026 81.40954) (end 106.599999 83.569801) (width 0.1778) (layer "F.Cu") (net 3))
 (segment (start 29.462017 83.569801) (end 27.02512 81.132904) (width 0.1778) (layer "F.Cu") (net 3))
 (segment (start 27.02512 68.21988) (end 29.21 66.035) (width 0.1778) (layer "F.Cu") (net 3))
 (segment (start 29.314921 83.924921) (end 111.777291 83.924921) (width 0.1778) (layer "F.Cu") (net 4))
 (segment (start 111.777291 83.924921) (end 112.75822 82.943992) (width 0.1778) (layer "F.Cu") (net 4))
 (segment (start 112.75822 82.943992) (end 112.75822 81.40954) (width 0.1778) (layer "F.Cu") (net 4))
 (segment (start 26.67 66.04) (end 26.67 81.28) (width 0.1778) (layer "F.Cu") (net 4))
 (segment (start 27.94 64.77) (end 26.67 66.04) (width 0.1778) (layer "F.Cu") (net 4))
 (segment (start 26.67 81.28) (end 29.314921 83.924921) (width 0.1778) (layer "F.Cu") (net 4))
 (segment (start 30.485 64.77) (end 27.94 64.77) (width 0.1778) (layer "F.Cu") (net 4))
 (segment (start 31.75 66.035) (end 30.485 64.77) (width 0.1778) (layer "F.Cu") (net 4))
 (segment (start 32.56026 53.46954) (end 32.56026 64.30526) (width 0.1778) (layer "F.Cu") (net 7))
 (segment (start 32.56026 64.30526) (end 34.29 66.035) (width 0.1778) (layer "F.Cu") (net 7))
 (segment (start 36.55822 53.46954) (end 36.55822 65.76322) (width 0.1778) (layer "F.Cu") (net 8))
 (segment (start 36.55822 65.76322) (end 36.83 66.035) (width 0.1778) (layer "F.Cu") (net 8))
 (segment (start 57.96026 45.84954) (end 39.37 64.4398) (width 0.1778) (layer "F.Cu") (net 11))
 (segment (start 39.37 64.4398) (end 39.37 66.035) (width 0.1778) (layer "F.Cu") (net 11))
 (segment (start 57.15 49.53) (end 59.77763 49.53) (width 0.1778) (layer "F.Cu") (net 10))
 (segment (start 61.95822 47.34941) (end 61.95822 45.84954) (width 0.1778) (layer "F.Cu") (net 10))
 (segment (start 59.77763 49.53) (end 61.95822 47.34941) (width 0.1778) (layer "F.Cu") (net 10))
 (segment (start 41.91 64.77) (end 57.15 49.53) (width 0.1778) (layer "F.Cu") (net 10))
 (segment (start 41.91 66.035) (end 41.91 64.77) (width 0.1778) (layer "F.Cu") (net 10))
 (segment (start 83.36026 53.46954) (end 57.01546 53.46954) (width 0.1778) (layer "F.Cu") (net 5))
 (segment (start 57.01546 53.46954) (end 44.45 66.035) (width 0.1778) (layer "F.Cu") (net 5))
 (segment (start 87.35822 55.003992) (end 85.212212 57.15) (width 0.1778) (layer "F.Cu") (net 6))
 (segment (start 85.212212 57.15) (end 55.875 57.15) (width 0.1778) (layer "F.Cu") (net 6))
 (segment (start 87.35822 53.46954) (end 87.35822 55.003992) (width 0.1778) (layer "F.Cu") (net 6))
 (segment (start 55.875 57.15) (end 46.99 66.035) (width 0.1778) (layer "F.Cu") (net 6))
 (segment (start 57.15 81.275) (end 59.530841 78.894159) (width 0.1778) (layer "F.Cu") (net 9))
 (segment (start 111.76 57.15) (end 119.38 57.15) (width 0.1778) (layer "F.Cu") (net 9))
 (segment (start 59.530841 78.894159) (end 90.015841 78.894159) (width 0.1778) (layer "F.Cu") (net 9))
 (segment (start 90.015841 78.894159) (end 111.76 57.15) (width 0.1778) (layer "F.Cu") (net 9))
 (segment (start 57.345961 78.539039) (end 54.61 81.275) (width 0.1778) (layer "F.Cu") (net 14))
 (segment (start 87.830961 78.539039) (end 57.345961 78.539039) (width 0.1778) (layer "F.Cu") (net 14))
 (segment (start 119.38 46.99) (end 87.830961 78.539039) (width 0.1778) (layer "F.Cu") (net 14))
 (segment (start 116.84 48.26) (end 86.916081 78.183919) (width 0.1778) (layer "F.Cu") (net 15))
 (segment (start 86.916081 78.183919) (end 55.161081 78.183919) (width 0.1778) (layer "F.Cu") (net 15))
 (segment (start 116.84 46.99) (end 116.84 48.26) (width 0.1778) (layer "F.Cu") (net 15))
 (segment (start 55.161081 78.183919) (end 52.07 81.275) (width 0.1778) (layer "F.Cu") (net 15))
 (segment (start 116.84 46.99) (end 119.38 44.45) (width 0.1778) (layer "F.Cu") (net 15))
 (segment (start 86.768985 77.828799) (end 52.976201 77.828799) (width 0.1778) (layer "F.Cu") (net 13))
 (segment (start 52.976201 77.828799) (end 49.53 81.275) (width 0.1778) (layer "F.Cu") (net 13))
 (segment (start 116.48488 48.112904) (end 86.768985 77.828799) (width 0.1778) (layer "F.Cu") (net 13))
 (segment (start 116.48488 44.80512) (end 116.48488 48.112904) (width 0.1778) (layer "F.Cu") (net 13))
 (segment (start 119.38 41.91) (end 116.48488 44.80512) (width 0.1778) (layer "F.Cu") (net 13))
 (segment (start 116.12976 42.62024) (end 116.12976 47.965808) (width 0.1778) (layer "F.Cu") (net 12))
 (segment (start 119.38 39.37) (end 116.12976 42.62024) (width 0.1778) (layer "F.Cu") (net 12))
 (segment (start 86.625568 77.47) (end 50.795 77.47) (width 0.1778) (layer "F.Cu") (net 12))
 (segment (start 50.795 77.47) (end 46.99 81.275) (width 0.1778) (layer "F.Cu") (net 12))
 (segment (start 116.12976 47.965808) (end 86.625568 77.47) (width 0.1778) (layer "F.Cu") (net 12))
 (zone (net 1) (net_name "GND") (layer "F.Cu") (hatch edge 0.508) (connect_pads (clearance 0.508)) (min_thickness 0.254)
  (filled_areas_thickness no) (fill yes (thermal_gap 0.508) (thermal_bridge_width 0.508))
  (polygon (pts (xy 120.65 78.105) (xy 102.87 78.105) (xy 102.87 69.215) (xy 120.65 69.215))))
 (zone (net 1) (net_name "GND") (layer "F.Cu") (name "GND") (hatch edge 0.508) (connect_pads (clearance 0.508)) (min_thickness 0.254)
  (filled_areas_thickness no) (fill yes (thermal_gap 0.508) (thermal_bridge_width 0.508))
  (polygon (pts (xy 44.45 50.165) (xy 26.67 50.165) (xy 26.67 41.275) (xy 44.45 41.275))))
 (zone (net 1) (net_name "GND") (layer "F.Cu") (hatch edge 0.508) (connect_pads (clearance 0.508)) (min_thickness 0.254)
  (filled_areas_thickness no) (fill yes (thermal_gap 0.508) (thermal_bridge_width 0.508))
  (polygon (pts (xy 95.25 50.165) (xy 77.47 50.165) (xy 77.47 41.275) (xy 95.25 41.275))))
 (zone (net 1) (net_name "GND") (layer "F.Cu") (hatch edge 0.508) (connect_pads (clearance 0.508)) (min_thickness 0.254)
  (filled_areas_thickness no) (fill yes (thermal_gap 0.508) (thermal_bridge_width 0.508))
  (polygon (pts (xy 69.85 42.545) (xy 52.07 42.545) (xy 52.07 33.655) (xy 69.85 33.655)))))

